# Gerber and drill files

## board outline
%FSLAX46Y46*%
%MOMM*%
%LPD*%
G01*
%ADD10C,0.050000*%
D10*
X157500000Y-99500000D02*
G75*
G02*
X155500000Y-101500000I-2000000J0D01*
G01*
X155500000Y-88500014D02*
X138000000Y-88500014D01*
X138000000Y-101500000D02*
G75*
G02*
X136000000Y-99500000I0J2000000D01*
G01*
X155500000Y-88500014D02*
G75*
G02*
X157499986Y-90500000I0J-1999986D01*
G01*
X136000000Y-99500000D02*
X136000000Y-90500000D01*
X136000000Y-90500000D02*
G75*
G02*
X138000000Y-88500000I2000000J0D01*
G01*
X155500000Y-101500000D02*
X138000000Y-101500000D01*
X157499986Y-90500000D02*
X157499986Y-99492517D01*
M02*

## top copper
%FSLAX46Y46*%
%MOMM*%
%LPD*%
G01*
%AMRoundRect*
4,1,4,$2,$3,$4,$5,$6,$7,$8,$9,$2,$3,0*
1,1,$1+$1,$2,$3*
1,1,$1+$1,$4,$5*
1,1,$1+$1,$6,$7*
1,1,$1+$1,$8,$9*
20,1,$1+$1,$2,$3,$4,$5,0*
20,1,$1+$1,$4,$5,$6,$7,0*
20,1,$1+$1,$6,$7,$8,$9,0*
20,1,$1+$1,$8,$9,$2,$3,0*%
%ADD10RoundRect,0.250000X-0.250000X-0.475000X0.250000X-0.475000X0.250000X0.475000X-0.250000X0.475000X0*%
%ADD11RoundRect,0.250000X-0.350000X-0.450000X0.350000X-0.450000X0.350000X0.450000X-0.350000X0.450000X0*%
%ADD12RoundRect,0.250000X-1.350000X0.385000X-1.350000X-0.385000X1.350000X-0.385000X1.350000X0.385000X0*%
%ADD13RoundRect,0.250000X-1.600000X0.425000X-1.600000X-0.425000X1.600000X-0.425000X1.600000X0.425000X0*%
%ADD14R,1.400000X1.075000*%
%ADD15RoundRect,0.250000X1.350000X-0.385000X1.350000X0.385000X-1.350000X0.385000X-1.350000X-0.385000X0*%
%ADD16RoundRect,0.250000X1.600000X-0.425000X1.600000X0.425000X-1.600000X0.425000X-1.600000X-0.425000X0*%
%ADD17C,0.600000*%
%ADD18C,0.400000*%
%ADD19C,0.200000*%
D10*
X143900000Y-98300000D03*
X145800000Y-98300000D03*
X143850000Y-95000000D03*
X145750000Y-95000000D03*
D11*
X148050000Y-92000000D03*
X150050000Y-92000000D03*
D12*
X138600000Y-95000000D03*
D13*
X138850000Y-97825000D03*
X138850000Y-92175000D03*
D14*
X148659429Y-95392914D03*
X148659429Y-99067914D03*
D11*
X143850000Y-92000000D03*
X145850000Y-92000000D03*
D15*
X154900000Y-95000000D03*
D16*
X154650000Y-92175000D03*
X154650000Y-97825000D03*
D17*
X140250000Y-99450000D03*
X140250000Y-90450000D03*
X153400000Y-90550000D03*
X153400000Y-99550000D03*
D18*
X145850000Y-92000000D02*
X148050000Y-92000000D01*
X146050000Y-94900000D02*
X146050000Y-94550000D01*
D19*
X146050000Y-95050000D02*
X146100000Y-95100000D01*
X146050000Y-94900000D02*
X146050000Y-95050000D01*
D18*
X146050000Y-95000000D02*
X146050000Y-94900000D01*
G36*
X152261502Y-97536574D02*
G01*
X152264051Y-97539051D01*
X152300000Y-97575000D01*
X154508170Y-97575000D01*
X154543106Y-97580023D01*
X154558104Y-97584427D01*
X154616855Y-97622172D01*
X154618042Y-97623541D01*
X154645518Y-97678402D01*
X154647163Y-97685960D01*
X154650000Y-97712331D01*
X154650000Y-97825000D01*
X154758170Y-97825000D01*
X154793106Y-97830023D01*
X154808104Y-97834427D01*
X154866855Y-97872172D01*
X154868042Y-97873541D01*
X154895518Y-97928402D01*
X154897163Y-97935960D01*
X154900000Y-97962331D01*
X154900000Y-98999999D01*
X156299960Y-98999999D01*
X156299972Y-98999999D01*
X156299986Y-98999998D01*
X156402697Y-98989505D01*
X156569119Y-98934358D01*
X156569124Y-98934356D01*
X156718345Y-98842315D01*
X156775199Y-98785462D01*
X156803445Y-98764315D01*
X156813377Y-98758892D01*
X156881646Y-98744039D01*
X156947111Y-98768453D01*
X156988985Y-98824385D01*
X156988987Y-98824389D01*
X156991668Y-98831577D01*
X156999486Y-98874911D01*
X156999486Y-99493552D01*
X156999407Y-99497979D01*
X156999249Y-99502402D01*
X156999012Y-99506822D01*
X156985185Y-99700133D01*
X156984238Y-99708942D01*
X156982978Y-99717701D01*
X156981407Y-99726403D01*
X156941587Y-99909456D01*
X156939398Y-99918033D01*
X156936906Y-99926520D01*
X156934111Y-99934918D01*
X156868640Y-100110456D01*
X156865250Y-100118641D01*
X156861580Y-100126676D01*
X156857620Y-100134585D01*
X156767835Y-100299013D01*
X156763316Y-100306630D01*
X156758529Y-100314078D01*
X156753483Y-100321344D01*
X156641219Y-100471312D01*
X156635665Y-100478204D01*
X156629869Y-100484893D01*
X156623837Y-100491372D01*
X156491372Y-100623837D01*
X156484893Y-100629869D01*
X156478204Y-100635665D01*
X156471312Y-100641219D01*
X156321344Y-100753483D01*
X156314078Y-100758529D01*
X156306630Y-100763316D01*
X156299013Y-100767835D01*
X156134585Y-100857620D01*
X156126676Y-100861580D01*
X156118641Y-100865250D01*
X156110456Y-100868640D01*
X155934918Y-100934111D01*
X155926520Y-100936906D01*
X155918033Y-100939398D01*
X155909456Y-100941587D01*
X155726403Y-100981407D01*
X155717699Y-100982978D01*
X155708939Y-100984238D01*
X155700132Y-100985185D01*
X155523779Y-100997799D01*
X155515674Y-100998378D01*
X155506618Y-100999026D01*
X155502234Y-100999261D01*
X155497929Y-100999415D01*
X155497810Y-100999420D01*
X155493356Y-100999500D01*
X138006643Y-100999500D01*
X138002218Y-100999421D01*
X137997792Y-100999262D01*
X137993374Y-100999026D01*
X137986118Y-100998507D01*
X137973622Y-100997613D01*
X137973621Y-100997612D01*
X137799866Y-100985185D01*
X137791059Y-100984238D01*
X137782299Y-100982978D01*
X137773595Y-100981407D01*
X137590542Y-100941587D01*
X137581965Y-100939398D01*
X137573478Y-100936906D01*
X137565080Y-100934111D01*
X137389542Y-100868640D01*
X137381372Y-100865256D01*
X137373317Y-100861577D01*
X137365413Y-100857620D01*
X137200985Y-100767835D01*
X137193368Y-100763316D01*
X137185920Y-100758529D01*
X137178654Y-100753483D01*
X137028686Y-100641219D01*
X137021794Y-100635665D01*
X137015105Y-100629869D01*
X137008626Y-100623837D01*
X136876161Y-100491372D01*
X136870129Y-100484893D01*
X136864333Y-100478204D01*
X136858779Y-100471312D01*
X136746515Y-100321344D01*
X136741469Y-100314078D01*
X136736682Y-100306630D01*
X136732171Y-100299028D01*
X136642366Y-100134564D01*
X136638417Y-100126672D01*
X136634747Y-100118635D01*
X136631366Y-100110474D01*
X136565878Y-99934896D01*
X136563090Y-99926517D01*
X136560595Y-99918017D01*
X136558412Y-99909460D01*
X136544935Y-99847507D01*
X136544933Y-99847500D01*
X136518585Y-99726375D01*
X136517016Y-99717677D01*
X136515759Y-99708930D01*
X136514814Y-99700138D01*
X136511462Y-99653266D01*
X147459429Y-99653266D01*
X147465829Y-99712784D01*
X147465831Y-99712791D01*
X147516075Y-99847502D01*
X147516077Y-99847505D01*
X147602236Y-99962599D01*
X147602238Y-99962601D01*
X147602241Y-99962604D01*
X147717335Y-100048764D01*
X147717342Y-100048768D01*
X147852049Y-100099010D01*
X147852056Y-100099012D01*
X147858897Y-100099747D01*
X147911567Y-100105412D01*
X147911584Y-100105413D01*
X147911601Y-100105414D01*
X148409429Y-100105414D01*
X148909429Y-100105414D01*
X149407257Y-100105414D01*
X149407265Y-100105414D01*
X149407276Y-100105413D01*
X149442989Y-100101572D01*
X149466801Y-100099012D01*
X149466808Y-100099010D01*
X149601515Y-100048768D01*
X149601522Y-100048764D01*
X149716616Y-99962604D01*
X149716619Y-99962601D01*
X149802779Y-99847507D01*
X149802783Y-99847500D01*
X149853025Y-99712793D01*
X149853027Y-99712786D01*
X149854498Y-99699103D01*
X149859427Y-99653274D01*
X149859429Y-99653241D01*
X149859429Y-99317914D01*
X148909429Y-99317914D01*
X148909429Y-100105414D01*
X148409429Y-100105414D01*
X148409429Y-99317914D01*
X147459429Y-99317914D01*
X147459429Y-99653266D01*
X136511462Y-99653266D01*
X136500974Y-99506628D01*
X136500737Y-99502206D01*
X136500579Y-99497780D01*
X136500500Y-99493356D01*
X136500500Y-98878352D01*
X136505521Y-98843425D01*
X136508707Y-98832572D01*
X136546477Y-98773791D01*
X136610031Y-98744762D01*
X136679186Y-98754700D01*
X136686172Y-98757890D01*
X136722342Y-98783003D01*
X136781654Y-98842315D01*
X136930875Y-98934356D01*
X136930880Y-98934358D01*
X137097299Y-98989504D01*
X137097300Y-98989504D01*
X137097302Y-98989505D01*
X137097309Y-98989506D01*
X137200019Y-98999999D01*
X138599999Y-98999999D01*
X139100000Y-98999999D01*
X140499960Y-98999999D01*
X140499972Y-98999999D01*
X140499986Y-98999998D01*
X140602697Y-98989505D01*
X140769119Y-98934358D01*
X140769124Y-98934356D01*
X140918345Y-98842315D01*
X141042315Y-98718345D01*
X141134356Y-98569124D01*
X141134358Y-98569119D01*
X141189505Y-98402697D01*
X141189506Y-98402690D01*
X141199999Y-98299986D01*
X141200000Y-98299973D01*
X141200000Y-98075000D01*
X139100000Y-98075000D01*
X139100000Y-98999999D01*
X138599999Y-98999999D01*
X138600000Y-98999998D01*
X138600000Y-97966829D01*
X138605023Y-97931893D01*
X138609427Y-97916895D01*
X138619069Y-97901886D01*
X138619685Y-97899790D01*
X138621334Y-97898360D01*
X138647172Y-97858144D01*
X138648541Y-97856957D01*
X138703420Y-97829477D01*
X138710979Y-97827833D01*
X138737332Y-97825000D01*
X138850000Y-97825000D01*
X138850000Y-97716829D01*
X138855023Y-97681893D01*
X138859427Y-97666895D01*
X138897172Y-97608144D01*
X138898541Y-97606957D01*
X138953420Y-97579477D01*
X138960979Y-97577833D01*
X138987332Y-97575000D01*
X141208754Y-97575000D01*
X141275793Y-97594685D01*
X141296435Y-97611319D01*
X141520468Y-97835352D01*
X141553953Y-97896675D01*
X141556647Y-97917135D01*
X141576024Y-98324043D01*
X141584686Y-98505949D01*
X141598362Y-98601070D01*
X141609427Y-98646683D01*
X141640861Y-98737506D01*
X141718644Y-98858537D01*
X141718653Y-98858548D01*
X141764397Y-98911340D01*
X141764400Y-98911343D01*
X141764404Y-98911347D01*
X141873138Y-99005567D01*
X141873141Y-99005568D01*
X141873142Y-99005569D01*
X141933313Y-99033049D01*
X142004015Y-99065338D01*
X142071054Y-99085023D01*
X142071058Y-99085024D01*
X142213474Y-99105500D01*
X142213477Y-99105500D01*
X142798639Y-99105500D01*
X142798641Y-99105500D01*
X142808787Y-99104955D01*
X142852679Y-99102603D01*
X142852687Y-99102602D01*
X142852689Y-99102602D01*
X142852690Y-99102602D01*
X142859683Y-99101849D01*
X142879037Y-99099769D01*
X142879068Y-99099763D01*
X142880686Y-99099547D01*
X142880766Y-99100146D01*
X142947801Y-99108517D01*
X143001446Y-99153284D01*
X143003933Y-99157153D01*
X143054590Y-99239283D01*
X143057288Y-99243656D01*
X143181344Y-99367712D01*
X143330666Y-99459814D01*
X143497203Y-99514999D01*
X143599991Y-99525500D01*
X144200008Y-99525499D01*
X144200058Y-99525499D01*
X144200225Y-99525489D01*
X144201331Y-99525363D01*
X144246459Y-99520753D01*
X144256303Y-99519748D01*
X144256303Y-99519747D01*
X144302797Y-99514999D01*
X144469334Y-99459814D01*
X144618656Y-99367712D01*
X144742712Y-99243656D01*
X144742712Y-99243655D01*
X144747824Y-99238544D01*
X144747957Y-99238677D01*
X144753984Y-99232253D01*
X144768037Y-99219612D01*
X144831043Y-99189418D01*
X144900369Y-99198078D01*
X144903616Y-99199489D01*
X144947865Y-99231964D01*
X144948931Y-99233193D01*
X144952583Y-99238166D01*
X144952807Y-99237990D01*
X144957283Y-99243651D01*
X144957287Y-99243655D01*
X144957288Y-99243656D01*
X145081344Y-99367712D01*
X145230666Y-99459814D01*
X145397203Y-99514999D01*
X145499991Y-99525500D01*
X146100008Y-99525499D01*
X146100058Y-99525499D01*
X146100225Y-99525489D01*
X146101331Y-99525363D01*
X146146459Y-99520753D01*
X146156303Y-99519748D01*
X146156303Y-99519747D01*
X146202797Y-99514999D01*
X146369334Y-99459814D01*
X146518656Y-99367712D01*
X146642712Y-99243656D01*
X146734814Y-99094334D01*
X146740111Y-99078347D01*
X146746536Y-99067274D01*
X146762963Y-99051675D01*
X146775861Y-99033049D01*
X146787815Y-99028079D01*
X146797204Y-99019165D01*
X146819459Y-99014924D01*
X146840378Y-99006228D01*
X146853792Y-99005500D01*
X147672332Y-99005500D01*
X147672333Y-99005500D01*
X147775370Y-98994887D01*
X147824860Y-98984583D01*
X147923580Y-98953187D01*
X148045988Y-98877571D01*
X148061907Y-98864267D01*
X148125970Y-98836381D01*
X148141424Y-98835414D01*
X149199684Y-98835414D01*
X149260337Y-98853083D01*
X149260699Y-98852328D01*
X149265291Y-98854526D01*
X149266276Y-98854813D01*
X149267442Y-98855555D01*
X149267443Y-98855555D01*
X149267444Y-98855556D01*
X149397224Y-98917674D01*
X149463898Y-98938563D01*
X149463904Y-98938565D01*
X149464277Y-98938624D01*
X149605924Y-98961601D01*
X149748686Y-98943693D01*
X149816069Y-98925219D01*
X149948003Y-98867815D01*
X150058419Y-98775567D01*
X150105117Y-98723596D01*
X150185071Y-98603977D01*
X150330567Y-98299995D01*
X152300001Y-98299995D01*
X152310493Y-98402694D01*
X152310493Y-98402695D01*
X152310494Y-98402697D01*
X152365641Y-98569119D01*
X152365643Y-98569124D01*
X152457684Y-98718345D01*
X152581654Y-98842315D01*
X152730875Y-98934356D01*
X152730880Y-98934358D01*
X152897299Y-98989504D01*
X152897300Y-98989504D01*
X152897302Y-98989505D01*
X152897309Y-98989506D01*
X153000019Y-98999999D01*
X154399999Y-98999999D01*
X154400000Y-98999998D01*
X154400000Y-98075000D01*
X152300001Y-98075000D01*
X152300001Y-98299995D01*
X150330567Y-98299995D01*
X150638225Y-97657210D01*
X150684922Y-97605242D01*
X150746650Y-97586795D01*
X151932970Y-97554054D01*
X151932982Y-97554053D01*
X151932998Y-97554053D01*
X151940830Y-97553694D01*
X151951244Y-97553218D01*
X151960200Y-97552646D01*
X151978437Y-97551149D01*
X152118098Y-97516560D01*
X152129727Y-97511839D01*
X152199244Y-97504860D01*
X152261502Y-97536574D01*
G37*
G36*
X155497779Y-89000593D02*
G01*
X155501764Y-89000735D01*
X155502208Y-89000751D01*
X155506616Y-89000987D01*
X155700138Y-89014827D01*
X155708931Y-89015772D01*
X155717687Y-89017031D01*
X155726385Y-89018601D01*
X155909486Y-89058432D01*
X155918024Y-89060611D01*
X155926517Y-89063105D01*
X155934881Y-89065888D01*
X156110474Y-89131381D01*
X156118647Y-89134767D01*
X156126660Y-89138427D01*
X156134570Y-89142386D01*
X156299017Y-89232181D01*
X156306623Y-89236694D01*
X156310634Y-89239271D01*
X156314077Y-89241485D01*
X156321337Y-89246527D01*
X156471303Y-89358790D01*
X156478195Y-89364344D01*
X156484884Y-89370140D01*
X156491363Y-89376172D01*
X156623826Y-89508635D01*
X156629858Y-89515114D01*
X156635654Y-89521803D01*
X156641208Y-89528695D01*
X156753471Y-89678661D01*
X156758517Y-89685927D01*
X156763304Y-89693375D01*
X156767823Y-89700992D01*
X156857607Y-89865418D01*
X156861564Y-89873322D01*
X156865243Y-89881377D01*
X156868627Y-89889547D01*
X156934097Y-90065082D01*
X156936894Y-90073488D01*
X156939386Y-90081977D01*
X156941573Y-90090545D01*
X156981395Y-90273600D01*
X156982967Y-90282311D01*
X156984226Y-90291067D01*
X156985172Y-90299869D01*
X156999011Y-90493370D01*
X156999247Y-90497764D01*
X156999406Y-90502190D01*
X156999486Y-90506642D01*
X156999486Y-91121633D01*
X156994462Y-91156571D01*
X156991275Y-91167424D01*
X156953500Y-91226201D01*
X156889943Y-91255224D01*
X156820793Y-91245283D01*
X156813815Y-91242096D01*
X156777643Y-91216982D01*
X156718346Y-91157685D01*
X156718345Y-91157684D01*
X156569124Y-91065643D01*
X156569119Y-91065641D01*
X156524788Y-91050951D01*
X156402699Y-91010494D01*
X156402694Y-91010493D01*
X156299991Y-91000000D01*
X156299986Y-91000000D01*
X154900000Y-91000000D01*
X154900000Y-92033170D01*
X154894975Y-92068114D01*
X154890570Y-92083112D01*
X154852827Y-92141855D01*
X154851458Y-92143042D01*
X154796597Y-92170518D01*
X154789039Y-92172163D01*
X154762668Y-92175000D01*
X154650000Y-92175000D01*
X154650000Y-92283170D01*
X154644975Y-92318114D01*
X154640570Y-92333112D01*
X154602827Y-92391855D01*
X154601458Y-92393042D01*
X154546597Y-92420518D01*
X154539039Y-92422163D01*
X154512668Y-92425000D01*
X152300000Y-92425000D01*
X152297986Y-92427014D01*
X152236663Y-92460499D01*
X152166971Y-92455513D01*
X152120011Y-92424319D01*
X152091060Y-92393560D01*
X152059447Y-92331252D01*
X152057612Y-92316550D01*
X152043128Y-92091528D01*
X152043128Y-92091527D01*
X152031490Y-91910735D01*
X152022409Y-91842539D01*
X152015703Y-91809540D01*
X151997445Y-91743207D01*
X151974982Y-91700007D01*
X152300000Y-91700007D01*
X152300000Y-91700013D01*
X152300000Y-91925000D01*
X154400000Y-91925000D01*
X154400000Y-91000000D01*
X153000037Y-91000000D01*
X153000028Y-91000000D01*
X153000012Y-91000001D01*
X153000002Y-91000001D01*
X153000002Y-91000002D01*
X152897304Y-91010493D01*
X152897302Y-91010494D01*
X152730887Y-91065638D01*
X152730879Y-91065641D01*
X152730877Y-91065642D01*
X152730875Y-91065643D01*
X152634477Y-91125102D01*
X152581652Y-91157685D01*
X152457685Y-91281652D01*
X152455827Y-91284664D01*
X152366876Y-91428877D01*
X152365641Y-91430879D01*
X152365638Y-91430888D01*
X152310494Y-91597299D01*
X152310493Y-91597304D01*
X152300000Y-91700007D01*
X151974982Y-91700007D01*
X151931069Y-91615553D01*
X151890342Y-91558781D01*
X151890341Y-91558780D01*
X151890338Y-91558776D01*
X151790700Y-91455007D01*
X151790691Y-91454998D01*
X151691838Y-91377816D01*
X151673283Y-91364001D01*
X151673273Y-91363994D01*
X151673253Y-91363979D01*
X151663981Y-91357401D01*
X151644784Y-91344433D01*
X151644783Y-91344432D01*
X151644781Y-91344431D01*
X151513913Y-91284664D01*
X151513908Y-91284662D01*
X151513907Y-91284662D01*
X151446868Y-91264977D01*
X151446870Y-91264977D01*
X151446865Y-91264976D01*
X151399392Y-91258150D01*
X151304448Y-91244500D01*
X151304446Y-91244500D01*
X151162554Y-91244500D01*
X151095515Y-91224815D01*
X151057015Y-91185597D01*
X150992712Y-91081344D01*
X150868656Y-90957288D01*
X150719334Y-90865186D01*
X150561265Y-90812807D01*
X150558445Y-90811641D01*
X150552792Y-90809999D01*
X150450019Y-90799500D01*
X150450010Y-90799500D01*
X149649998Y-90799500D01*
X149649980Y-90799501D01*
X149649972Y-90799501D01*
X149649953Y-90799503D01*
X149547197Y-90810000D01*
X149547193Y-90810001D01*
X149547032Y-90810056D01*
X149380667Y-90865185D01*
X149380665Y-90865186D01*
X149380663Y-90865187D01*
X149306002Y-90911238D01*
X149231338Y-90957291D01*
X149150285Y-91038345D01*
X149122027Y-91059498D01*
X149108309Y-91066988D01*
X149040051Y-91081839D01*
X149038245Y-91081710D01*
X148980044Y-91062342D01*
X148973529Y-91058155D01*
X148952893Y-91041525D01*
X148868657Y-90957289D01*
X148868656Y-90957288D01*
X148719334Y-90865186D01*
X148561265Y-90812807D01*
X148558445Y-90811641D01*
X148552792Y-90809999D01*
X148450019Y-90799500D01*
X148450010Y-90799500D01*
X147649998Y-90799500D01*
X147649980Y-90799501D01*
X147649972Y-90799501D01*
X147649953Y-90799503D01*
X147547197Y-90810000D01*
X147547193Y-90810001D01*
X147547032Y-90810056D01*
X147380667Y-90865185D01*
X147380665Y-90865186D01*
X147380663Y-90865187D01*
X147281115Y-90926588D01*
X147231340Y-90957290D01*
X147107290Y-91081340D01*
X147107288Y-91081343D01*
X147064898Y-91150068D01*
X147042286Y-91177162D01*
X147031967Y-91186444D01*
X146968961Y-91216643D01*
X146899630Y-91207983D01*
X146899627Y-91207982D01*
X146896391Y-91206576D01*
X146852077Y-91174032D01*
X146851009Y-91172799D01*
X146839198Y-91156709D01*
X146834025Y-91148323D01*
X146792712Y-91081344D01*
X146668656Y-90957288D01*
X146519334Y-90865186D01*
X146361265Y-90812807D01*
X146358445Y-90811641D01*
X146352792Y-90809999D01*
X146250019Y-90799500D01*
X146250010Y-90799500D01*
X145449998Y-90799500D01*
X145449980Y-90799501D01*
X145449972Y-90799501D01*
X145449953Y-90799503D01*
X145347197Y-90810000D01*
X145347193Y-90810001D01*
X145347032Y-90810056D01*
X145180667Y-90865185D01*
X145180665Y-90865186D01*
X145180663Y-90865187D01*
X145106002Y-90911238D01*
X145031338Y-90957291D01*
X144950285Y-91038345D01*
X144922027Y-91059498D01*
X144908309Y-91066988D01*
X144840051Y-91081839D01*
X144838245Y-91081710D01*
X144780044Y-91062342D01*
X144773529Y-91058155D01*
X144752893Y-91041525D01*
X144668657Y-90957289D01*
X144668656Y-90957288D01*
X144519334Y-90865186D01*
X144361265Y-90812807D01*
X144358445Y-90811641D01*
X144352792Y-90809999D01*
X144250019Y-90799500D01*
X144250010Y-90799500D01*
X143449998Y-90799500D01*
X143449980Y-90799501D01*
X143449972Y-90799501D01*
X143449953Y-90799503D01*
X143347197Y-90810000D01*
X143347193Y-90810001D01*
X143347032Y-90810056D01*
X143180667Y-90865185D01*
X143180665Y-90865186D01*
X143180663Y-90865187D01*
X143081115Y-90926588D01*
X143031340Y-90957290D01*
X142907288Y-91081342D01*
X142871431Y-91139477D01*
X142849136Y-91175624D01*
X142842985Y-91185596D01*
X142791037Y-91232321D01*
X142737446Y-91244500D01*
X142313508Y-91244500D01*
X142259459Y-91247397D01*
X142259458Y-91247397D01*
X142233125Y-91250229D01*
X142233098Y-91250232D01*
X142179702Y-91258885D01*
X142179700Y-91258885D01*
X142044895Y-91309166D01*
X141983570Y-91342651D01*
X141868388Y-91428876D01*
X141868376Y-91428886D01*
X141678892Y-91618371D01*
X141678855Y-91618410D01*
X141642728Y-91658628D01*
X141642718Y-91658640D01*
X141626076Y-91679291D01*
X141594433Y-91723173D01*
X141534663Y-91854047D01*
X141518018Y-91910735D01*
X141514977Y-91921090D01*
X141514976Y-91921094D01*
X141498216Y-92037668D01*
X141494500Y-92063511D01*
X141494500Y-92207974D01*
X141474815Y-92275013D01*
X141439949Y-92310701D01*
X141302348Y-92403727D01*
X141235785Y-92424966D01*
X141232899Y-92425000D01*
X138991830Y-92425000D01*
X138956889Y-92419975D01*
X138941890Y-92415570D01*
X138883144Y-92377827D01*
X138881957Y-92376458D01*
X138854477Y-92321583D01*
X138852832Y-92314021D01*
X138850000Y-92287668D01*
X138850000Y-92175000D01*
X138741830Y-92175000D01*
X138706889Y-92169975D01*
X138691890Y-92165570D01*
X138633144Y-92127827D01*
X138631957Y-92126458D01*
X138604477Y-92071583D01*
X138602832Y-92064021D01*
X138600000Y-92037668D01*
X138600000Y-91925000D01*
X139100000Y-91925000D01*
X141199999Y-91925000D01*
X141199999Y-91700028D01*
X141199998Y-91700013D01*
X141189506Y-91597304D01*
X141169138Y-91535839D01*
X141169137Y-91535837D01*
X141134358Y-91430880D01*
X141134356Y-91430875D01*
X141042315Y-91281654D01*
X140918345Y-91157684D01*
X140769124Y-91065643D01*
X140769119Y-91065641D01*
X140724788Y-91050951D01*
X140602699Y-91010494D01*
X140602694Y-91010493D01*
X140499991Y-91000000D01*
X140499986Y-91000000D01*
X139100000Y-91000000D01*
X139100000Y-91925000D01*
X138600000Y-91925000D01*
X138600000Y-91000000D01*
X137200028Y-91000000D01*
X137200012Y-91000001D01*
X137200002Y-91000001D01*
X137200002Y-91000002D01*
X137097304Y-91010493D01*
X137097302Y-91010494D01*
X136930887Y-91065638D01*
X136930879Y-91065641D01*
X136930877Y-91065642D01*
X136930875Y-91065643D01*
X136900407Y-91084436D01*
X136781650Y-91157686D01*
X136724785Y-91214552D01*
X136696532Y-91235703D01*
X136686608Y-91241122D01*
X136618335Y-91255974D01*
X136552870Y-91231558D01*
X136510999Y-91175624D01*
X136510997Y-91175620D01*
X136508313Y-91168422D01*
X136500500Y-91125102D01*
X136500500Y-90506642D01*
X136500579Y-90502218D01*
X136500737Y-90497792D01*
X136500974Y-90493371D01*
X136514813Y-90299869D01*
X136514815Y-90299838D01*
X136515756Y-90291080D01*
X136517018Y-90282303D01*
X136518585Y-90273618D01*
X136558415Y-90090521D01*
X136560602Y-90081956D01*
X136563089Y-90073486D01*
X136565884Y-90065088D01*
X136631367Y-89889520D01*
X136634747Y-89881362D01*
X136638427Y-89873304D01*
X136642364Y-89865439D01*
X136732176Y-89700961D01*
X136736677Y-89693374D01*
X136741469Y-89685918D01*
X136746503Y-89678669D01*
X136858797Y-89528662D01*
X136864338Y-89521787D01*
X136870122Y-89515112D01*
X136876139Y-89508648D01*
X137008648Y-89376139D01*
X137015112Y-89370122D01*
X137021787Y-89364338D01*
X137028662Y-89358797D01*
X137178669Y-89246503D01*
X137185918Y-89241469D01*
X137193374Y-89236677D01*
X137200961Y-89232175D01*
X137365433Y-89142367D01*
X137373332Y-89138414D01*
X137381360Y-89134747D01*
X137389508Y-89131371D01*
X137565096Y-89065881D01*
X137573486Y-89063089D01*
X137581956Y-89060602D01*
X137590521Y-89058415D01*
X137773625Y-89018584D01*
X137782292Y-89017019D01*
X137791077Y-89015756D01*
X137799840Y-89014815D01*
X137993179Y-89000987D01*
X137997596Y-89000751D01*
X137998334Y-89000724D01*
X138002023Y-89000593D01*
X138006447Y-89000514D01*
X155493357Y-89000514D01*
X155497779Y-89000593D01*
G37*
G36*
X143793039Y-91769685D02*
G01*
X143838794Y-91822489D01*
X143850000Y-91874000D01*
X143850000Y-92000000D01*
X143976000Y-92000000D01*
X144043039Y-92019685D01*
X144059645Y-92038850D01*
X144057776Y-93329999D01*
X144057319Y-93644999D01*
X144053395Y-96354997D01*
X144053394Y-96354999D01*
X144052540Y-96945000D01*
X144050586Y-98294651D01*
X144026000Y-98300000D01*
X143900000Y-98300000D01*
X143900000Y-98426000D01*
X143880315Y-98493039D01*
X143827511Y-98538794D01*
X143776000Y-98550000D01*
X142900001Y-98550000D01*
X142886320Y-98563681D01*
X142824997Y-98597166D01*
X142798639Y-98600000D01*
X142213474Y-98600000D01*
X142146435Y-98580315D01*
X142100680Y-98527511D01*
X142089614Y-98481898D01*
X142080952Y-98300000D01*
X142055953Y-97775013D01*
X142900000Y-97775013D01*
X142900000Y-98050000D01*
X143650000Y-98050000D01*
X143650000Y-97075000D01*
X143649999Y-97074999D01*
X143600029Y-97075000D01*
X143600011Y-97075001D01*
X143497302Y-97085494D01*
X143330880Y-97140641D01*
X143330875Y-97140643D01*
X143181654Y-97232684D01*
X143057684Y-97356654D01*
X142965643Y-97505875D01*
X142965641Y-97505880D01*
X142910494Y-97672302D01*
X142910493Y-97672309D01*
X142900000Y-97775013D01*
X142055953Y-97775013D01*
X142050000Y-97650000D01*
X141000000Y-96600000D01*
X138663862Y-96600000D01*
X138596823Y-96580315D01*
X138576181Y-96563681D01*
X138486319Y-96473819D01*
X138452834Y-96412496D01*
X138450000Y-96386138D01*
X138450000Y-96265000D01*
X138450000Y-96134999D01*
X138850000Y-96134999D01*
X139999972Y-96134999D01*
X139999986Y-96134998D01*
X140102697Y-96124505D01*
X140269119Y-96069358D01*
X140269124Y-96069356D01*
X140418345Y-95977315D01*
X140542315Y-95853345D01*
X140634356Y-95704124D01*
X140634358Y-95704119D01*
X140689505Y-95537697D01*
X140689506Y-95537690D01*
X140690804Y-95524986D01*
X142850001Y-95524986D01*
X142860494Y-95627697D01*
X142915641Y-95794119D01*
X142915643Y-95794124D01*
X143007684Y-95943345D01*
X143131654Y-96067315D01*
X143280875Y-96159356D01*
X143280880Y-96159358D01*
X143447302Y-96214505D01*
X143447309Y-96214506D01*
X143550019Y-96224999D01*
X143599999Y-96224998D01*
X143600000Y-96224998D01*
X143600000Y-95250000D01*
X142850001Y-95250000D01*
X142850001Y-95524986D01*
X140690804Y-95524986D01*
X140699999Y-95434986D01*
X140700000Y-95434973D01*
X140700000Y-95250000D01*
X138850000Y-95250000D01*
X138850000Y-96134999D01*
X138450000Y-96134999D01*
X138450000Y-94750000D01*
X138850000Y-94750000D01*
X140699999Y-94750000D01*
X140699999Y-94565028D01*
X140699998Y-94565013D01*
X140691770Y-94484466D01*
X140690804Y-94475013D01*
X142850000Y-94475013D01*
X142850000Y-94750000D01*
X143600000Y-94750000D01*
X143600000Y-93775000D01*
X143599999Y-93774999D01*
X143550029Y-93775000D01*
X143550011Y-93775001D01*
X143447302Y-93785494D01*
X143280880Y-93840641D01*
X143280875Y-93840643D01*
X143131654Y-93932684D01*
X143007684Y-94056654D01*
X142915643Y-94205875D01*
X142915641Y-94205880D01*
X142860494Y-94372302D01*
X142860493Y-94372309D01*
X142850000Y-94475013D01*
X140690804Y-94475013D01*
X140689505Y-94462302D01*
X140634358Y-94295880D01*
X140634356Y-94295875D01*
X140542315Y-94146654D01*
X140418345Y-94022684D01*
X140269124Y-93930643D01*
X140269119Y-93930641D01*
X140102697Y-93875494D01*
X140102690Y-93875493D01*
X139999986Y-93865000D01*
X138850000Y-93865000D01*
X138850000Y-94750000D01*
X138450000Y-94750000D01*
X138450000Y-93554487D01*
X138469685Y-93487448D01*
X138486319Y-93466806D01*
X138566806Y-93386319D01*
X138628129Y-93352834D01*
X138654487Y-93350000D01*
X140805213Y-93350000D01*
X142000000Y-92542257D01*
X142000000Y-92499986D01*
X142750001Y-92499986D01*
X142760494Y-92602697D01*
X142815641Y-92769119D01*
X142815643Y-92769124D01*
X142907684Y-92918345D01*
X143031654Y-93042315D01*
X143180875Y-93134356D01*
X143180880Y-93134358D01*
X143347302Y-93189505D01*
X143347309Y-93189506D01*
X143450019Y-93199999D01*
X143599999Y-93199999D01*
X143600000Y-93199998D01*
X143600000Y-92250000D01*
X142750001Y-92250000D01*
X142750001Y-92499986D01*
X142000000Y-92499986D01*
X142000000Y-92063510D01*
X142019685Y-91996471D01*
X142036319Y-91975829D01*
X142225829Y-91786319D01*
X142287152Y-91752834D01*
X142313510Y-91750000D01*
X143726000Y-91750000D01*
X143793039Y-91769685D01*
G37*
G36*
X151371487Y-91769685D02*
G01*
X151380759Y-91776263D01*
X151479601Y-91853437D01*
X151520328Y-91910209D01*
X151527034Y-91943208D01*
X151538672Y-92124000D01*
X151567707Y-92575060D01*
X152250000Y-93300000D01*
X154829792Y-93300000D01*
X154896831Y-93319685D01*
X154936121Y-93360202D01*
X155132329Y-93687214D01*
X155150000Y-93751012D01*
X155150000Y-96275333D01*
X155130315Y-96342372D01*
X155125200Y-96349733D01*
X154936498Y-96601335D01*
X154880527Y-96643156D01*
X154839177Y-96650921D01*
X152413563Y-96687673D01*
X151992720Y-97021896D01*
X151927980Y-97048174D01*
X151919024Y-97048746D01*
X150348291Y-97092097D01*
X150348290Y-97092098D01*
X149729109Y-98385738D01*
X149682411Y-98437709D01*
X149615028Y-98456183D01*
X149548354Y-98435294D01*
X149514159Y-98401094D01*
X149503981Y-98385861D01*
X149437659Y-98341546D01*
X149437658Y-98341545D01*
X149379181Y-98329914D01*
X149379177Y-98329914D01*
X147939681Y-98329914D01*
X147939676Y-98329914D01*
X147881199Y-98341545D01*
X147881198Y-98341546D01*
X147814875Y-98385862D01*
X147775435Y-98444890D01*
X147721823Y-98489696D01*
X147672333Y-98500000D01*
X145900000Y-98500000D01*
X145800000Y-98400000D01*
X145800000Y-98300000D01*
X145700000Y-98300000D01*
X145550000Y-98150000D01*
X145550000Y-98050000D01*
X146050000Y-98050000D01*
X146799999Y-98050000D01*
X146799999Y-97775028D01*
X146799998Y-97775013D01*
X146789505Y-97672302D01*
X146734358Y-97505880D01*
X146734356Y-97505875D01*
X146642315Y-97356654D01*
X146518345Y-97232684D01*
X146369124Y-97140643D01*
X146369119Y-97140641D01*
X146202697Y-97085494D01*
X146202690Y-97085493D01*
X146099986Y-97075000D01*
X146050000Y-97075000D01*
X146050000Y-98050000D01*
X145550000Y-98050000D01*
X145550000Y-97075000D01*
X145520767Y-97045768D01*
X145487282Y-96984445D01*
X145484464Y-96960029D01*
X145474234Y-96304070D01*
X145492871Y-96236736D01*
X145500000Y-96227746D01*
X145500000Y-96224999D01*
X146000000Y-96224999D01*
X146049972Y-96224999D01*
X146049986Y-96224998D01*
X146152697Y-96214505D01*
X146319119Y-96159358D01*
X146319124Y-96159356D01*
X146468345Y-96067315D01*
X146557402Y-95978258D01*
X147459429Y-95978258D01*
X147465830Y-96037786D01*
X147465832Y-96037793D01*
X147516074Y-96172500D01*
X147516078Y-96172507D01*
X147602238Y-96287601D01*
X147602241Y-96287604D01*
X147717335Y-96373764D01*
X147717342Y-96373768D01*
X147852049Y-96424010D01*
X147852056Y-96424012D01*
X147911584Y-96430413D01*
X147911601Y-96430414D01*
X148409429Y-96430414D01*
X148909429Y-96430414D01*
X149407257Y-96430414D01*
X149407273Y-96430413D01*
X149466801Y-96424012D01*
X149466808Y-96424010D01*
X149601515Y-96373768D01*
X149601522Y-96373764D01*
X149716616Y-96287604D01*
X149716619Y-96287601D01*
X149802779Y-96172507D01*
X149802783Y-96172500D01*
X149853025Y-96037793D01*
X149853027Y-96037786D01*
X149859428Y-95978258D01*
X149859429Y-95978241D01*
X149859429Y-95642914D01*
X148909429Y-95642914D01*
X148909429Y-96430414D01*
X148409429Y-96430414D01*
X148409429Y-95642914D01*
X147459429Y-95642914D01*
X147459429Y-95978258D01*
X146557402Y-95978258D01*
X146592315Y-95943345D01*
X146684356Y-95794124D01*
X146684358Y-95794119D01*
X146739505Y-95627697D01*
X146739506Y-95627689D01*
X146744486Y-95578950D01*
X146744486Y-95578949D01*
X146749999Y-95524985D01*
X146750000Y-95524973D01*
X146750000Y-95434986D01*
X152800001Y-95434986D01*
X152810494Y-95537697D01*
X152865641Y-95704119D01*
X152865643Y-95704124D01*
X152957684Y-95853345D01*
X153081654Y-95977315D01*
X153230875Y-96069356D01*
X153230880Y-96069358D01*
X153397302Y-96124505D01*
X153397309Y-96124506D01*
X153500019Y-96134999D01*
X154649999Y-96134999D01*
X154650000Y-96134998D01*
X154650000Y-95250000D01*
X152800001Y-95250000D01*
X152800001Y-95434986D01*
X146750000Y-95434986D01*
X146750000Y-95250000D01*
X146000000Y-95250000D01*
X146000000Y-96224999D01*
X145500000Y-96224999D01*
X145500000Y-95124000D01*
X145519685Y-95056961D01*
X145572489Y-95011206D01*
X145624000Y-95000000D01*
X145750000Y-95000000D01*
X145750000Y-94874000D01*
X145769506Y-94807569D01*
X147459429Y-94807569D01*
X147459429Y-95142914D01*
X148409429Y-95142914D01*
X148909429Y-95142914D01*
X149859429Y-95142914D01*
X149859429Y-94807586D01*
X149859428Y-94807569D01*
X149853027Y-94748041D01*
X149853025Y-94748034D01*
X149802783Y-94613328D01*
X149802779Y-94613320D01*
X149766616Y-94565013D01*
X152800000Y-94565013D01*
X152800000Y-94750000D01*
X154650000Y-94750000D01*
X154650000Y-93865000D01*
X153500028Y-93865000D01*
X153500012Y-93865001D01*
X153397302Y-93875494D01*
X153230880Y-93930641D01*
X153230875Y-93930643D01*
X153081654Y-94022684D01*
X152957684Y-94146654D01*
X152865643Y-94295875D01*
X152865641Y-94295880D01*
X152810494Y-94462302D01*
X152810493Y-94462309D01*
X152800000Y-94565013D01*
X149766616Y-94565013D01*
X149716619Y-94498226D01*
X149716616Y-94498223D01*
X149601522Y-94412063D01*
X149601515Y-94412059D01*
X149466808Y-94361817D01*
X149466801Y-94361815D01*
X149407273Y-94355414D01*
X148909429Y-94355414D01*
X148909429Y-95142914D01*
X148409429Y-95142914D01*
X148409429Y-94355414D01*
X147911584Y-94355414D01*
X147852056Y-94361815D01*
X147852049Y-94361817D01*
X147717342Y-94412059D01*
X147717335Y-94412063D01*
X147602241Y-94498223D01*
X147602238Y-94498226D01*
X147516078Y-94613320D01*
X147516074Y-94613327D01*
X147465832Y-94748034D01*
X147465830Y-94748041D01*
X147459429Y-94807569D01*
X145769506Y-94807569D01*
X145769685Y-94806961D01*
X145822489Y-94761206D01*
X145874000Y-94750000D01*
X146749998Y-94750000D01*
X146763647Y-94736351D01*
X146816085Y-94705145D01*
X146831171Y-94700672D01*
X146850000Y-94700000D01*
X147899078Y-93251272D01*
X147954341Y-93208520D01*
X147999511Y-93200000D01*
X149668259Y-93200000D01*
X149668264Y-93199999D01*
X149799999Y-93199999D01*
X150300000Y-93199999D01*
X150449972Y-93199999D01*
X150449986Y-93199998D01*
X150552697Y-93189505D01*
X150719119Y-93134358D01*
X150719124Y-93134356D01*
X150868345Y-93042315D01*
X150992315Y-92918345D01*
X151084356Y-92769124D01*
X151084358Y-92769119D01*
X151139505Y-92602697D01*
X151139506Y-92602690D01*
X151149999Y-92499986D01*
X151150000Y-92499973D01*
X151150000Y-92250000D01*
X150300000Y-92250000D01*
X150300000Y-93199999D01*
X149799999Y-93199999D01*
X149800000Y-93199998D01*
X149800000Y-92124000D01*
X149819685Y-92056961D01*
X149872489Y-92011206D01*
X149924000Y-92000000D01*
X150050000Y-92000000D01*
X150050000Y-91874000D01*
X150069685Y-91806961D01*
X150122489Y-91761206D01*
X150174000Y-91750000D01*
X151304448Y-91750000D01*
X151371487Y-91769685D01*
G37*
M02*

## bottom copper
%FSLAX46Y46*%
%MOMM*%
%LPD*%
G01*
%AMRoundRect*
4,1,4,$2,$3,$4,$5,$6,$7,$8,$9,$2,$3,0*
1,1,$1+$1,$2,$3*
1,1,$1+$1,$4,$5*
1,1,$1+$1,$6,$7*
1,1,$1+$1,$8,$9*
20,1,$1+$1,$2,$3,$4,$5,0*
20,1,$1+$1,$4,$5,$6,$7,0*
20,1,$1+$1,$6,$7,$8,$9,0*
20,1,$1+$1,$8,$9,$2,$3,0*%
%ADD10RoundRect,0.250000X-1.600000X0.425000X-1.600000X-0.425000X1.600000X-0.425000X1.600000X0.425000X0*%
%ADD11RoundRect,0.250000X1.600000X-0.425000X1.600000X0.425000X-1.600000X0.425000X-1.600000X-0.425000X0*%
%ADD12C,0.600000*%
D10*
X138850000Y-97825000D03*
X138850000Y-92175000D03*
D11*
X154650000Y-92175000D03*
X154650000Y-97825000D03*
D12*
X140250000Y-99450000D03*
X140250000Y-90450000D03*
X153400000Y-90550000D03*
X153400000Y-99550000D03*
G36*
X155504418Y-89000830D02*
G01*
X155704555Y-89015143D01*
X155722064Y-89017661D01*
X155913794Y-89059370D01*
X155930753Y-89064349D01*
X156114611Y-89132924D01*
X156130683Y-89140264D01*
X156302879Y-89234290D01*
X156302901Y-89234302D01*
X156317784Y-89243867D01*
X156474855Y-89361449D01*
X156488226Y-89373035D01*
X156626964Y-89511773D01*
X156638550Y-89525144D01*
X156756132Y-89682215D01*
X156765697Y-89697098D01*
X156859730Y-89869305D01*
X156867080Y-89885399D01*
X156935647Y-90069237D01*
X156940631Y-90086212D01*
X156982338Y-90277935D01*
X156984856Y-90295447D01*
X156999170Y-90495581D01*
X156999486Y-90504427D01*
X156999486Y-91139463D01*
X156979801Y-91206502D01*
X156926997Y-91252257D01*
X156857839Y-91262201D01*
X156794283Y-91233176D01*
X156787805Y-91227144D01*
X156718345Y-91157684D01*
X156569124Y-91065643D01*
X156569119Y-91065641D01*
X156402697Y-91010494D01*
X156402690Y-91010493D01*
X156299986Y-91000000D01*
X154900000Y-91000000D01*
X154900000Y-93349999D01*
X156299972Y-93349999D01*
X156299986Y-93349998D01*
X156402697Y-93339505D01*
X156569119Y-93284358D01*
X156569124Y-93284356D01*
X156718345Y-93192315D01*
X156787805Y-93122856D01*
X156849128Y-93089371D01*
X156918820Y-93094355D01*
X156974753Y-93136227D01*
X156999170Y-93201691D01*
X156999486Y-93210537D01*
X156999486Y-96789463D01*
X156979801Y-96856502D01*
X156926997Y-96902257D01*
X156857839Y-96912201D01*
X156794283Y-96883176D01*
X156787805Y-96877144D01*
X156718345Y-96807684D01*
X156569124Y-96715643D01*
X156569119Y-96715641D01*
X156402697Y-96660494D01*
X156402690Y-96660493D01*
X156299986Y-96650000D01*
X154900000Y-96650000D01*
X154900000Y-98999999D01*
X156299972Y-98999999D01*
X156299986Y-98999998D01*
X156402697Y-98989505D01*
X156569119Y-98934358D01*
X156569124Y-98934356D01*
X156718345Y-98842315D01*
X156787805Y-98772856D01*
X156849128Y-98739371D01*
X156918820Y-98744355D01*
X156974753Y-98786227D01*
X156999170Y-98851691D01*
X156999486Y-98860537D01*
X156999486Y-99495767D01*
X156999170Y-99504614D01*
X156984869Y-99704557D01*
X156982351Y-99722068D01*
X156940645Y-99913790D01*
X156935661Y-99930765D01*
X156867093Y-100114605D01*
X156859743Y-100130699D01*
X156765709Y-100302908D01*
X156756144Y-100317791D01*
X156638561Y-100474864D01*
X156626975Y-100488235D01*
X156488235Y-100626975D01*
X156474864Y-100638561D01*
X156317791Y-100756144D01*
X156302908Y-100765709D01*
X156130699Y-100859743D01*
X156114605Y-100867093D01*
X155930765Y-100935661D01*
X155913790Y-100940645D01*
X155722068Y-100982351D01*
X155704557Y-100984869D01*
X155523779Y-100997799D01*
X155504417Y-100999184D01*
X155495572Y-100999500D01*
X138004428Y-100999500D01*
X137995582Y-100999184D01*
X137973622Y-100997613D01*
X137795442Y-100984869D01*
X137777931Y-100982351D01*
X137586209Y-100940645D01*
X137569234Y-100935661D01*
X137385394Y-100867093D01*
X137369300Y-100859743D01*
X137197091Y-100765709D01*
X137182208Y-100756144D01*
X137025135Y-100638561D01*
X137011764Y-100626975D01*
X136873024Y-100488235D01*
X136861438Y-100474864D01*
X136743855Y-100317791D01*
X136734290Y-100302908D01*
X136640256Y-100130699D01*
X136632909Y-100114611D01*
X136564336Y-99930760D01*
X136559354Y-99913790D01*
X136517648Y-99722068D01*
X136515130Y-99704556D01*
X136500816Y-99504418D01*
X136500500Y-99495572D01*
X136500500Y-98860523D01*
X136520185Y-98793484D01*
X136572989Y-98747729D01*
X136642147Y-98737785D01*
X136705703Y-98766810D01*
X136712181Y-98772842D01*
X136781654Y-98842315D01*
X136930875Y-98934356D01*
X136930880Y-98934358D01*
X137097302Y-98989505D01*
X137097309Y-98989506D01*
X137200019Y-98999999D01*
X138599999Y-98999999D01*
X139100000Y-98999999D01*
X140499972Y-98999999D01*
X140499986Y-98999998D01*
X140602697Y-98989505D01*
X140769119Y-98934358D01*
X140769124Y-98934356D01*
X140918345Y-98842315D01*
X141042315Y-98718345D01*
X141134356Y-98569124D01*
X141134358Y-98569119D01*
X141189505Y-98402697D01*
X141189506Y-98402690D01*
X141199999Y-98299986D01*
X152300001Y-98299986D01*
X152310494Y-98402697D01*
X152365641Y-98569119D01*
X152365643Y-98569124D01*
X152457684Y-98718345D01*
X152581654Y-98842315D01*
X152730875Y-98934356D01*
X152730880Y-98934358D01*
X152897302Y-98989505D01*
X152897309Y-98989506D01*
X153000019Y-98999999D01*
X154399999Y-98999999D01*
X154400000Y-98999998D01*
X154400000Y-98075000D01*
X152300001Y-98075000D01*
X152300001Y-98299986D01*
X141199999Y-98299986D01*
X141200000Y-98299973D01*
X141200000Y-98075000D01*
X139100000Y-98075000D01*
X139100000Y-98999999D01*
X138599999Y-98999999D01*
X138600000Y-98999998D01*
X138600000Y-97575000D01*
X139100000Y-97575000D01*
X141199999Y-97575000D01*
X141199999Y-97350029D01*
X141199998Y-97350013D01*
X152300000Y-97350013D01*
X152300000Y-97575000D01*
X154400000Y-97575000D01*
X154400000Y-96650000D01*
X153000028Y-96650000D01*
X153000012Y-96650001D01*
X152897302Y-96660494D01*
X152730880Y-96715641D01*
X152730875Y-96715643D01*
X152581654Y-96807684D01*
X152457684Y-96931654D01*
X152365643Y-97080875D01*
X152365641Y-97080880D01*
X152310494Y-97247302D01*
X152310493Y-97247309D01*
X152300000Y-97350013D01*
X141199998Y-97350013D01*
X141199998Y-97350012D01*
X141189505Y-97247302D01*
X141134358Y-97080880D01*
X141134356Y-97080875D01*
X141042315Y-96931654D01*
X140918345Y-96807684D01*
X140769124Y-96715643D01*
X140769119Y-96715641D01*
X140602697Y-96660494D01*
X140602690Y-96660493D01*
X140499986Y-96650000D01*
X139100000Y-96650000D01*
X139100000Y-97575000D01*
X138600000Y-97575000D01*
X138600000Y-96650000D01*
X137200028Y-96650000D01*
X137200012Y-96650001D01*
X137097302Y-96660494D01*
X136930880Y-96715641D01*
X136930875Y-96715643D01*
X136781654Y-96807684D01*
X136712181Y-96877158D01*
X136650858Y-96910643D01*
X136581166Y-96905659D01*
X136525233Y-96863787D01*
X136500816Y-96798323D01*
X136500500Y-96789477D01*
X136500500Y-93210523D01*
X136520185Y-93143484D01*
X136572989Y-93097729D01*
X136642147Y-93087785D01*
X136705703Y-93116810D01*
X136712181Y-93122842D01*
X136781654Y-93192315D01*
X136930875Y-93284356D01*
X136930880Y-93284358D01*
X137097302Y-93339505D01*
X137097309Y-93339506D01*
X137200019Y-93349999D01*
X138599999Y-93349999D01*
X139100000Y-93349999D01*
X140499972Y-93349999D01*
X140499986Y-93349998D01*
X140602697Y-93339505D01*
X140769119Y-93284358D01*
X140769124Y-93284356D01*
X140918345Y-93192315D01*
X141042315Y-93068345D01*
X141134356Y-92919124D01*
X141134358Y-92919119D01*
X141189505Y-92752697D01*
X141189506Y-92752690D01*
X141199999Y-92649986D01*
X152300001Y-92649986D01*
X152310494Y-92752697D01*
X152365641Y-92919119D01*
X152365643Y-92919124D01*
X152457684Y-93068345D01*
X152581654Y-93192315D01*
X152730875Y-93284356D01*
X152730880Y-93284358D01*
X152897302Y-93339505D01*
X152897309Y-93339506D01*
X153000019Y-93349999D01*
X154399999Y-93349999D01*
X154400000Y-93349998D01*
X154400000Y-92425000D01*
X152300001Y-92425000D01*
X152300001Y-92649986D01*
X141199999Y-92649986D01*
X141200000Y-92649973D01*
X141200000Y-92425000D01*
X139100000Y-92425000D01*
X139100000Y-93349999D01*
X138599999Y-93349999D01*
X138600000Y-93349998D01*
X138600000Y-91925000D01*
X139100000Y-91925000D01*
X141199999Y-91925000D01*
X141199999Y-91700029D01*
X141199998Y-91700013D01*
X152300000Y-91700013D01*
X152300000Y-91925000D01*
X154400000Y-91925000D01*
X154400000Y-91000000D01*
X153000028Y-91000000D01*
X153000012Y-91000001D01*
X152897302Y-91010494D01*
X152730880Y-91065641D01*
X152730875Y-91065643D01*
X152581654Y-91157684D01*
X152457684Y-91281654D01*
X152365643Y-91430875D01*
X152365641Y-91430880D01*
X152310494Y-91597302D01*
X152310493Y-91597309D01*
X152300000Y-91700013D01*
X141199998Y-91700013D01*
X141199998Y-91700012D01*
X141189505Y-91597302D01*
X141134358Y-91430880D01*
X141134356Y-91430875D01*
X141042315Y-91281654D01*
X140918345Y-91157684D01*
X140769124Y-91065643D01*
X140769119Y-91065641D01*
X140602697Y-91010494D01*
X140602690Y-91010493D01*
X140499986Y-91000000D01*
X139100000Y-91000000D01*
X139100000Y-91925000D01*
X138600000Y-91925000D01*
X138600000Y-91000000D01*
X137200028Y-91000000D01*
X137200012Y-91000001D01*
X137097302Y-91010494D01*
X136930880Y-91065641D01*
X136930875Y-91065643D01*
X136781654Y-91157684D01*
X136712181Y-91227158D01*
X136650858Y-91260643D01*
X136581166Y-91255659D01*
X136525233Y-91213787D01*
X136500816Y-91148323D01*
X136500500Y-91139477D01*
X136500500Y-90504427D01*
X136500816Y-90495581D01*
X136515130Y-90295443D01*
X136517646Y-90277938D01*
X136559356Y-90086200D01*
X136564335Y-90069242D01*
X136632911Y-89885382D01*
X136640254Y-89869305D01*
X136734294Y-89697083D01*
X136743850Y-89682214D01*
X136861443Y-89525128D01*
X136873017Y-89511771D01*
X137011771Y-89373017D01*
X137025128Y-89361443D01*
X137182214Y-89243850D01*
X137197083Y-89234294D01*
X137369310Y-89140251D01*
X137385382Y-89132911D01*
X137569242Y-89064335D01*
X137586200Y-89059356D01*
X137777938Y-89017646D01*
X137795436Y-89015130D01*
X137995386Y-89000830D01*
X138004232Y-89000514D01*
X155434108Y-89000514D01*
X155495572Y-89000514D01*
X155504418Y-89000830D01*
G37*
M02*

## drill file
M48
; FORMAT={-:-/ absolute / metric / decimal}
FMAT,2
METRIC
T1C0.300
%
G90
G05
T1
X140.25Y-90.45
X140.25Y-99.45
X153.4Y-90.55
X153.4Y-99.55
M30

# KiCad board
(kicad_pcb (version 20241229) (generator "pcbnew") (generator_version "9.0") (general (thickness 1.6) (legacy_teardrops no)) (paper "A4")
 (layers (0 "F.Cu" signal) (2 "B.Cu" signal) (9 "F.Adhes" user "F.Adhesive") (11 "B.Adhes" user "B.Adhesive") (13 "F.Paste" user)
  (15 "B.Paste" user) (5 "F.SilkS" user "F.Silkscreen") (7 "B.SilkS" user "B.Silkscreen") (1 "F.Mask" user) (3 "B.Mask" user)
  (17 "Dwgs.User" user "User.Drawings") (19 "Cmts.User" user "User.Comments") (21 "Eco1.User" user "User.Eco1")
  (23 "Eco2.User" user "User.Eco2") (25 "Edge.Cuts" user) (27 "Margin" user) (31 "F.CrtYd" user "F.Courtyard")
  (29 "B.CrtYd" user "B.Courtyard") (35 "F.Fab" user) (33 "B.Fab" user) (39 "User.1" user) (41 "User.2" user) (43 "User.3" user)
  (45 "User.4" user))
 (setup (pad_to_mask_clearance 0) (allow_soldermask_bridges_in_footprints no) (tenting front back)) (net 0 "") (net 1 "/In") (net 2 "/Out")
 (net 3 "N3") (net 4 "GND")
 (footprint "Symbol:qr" (layer "F.Cu") (at 146.267513 95.7586)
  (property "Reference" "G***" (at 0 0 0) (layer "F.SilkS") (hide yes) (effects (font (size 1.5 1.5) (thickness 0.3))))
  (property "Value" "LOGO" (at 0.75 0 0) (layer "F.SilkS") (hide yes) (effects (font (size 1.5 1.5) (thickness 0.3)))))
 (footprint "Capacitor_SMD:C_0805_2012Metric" (layer "F.Cu") (at 144.85 98.3)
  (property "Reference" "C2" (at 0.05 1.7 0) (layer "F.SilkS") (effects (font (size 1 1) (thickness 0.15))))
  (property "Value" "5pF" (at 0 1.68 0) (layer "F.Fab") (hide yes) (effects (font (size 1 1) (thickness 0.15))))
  (pad "1" smd roundrect (at -0.95 0) (size 1 1.45) (layers "F.Cu" "F.Mask" "F.Paste") (roundrect_rratio 0.25) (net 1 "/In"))
  (pad "2" smd roundrect (at 0.95 0) (size 1 1.45) (layers "F.Cu" "F.Mask" "F.Paste") (roundrect_rratio 0.25) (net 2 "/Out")))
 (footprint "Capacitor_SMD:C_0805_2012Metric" (layer "F.Cu") (at 144.8 95)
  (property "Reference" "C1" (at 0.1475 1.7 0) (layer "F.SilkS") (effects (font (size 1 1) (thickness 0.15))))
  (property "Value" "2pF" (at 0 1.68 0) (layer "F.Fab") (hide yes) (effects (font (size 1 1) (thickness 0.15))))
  (pad "1" smd roundrect (at -0.95 0) (size 1 1.45) (layers "F.Cu" "F.Mask" "F.Paste") (roundrect_rratio 0.25) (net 1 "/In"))
  (pad "2" smd roundrect (at 0.95 0) (size 1 1.45) (layers "F.Cu" "F.Mask" "F.Paste") (roundrect_rratio 0.25) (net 2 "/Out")))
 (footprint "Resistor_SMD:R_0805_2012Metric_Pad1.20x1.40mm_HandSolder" (layer "F.Cu") (at 149.05 92)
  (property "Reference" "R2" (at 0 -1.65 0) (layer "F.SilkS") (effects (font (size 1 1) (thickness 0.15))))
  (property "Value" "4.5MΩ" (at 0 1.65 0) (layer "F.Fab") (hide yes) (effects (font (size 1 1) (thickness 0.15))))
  (pad "1" smd roundrect (at -1 0) (size 1.2 1.4) (layers "F.Cu" "F.Mask" "F.Paste") (roundrect_rratio 0.208333) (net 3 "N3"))
  (pad "2" smd roundrect (at 1 0) (size 1.2 1.4) (layers "F.Cu" "F.Mask" "F.Paste") (roundrect_rratio 0.208333) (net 2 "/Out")))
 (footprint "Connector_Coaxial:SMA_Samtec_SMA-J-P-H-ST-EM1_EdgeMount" (layer "F.Cu") (at 138.6 95 180)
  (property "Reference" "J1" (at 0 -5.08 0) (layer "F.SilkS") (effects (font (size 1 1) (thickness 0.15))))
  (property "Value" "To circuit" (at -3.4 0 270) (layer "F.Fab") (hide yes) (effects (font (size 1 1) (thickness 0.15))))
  (pad "1" smd roundrect (at 0 0 270) (size 1.27 3.2) (layers "F.Cu" "F.Mask") (roundrect_rratio 0.1968503937) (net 1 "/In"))
  (pad "2" smd roundrect (at -0.25 -2.825 270) (size 1.35 3.7) (layers "F.Cu" "F.Mask") (roundrect_rratio 0.1851851852) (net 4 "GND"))
  (pad "2" smd roundrect (at -0.25 -2.825 270) (size 1.35 3.7) (layers "B.Cu" "B.Mask") (roundrect_rratio 0.1851851852) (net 4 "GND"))
  (pad "2" smd roundrect (at -0.25 2.825 270) (size 1.35 3.7) (layers "F.Cu" "F.Mask") (roundrect_rratio 0.1851851852) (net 4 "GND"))
  (pad "2" smd roundrect (at -0.25 2.825 270) (size 1.35 3.7) (layers "B.Cu" "B.Mask") (roundrect_rratio 0.1851851852) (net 4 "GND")))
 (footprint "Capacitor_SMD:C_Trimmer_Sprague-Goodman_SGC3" (layer "F.Cu") (at 148.659429 97.230414 -90)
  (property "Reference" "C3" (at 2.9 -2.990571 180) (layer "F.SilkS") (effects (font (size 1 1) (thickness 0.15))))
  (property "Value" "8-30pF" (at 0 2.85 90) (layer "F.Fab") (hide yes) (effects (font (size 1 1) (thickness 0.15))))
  (pad "1" smd rect (at -1.8375 0 270) (size 1.075 1.4) (layers "F.Cu" "F.Mask" "F.Paste") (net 2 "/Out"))
  (pad "2" smd rect (at 1.8375 0 270) (size 1.075 1.4) (layers "F.Cu" "F.Mask" "F.Paste") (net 4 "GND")))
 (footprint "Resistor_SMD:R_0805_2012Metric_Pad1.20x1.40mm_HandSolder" (layer "F.Cu") (at 144.85 92)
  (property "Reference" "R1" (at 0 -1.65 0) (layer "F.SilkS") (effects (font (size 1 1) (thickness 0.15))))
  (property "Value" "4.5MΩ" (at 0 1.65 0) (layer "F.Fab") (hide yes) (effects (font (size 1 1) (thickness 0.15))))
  (pad "1" smd roundrect (at -1 0) (size 1.2 1.4) (layers "F.Cu" "F.Mask" "F.Paste") (roundrect_rratio 0.208333) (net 1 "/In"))
  (pad "2" smd roundrect (at 1 0) (size 1.2 1.4) (layers "F.Cu" "F.Mask" "F.Paste") (roundrect_rratio 0.208333) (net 3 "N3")))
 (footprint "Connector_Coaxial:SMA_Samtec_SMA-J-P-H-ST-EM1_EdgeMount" (layer "F.Cu") (at 154.9 95)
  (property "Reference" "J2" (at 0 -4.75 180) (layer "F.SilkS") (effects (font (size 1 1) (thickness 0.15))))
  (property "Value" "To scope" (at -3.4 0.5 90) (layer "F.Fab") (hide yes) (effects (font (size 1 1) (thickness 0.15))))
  (pad "1" smd roundrect (at 0 0 90) (size 1.27 3.2) (layers "F.Cu" "F.Mask") (roundrect_rratio 0.1968503937) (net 2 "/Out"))
  (pad "2" smd roundrect (at -0.25 -2.825 90) (size 1.35 3.7) (layers "F.Cu" "F.Mask") (roundrect_rratio 0.1851851852) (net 4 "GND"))
  (pad "2" smd roundrect (at -0.25 -2.825 90) (size 1.35 3.7) (layers "B.Cu" "B.Mask") (roundrect_rratio 0.1851851852) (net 4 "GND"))
  (pad "2" smd roundrect (at -0.25 2.825 90) (size 1.35 3.7) (layers "F.Cu" "F.Mask") (roundrect_rratio 0.1851851852) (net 4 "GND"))
  (pad "2" smd roundrect (at -0.25 2.825 90) (size 1.35 3.7) (layers "B.Cu" "B.Mask") (roundrect_rratio 0.1851851852) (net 4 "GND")))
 (gr_arc (start 157.5 99.5) (mid 156.914214 100.914214) (end 155.5 101.5) (stroke (width 0.05) (type solid)) (layer "Edge.Cuts"))
 (gr_line (start 155.5 88.500014) (end 138 88.500014) (stroke (width 0.05) (type default)) (layer "Edge.Cuts"))
 (gr_arc (start 138 101.5) (mid 136.585786 100.914214) (end 136 99.5) (stroke (width 0.05) (type default)) (layer "Edge.Cuts"))
 (gr_arc (start 155.5 88.500014) (mid 156.914204 89.085796) (end 157.499986 90.5) (stroke (width 0.05) (type default)) (layer "Edge.Cuts"))
 (gr_line (start 136 99.5) (end 136 90.5) (stroke (width 0.05) (type default)) (layer "Edge.Cuts"))
 (gr_arc (start 136 90.5) (mid 136.585786 89.085786) (end 138 88.5) (stroke (width 0.05) (type solid)) (layer "Edge.Cuts"))
 (gr_line (start 155.5 101.5) (end 138 101.5) (stroke (width 0.05) (type default)) (layer "Edge.Cuts"))
 (gr_line (start 157.499986 90.5) (end 157.499986 99.492517) (stroke (width 0.05) (type default)) (layer "Edge.Cuts"))
 (via (at 140.25 99.45) (size 0.6) (drill 0.3) (layers "F.Cu" "B.Cu") (free yes) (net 4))
 (via (at 140.25 90.45) (size 0.6) (drill 0.3) (layers "F.Cu" "B.Cu") (free yes) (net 4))
 (via (at 153.4 90.55) (size 0.6) (drill 0.3) (layers "F.Cu" "B.Cu") (free yes) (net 4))
 (via (at 153.4 99.55) (size 0.6) (drill 0.3) (layers "F.Cu" "B.Cu") (free yes) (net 4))
 (segment (start 145.85 92) (end 148.05 92) (width 0.4) (layer "F.Cu") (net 3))
 (segment (start 146.05 94.9) (end 146.05 94.55) (width 0.4) (layer "F.Cu") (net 2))
 (segment (start 146.05 95.05) (end 146.1 95.1) (width 0.2) (layer "F.Cu") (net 2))
 (segment (start 146.05 94.9) (end 146.05 95.05) (width 0.2) (layer "F.Cu") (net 2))
 (segment (start 146.05 95) (end 146.05 94.9) (width 0.4) (layer "F.Cu") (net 2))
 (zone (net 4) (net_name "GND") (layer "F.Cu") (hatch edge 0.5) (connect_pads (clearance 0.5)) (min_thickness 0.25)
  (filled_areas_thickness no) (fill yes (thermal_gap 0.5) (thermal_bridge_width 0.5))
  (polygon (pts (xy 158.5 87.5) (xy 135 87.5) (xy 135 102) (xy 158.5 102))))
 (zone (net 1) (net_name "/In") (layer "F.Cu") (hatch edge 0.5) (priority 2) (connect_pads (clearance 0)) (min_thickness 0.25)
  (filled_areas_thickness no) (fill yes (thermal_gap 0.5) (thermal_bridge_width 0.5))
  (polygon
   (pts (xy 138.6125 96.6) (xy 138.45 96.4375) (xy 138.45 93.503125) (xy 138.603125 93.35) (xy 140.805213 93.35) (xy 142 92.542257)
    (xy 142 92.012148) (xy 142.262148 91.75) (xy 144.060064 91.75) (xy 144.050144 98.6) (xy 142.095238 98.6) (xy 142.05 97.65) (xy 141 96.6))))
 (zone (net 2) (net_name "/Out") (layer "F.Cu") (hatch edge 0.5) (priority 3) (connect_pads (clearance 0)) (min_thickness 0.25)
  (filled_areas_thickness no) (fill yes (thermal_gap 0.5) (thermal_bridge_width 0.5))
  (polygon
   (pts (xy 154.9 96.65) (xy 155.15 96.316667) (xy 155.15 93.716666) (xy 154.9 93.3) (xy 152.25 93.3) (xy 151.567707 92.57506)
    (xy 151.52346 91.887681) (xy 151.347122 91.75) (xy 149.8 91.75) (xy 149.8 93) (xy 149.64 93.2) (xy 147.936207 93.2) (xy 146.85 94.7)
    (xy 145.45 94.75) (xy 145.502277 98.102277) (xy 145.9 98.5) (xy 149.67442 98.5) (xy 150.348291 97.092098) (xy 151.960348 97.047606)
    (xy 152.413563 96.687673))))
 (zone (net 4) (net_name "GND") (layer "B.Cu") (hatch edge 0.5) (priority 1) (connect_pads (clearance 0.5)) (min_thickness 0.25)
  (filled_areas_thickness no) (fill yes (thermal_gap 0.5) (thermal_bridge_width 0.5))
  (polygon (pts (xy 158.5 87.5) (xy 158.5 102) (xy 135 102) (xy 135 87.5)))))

